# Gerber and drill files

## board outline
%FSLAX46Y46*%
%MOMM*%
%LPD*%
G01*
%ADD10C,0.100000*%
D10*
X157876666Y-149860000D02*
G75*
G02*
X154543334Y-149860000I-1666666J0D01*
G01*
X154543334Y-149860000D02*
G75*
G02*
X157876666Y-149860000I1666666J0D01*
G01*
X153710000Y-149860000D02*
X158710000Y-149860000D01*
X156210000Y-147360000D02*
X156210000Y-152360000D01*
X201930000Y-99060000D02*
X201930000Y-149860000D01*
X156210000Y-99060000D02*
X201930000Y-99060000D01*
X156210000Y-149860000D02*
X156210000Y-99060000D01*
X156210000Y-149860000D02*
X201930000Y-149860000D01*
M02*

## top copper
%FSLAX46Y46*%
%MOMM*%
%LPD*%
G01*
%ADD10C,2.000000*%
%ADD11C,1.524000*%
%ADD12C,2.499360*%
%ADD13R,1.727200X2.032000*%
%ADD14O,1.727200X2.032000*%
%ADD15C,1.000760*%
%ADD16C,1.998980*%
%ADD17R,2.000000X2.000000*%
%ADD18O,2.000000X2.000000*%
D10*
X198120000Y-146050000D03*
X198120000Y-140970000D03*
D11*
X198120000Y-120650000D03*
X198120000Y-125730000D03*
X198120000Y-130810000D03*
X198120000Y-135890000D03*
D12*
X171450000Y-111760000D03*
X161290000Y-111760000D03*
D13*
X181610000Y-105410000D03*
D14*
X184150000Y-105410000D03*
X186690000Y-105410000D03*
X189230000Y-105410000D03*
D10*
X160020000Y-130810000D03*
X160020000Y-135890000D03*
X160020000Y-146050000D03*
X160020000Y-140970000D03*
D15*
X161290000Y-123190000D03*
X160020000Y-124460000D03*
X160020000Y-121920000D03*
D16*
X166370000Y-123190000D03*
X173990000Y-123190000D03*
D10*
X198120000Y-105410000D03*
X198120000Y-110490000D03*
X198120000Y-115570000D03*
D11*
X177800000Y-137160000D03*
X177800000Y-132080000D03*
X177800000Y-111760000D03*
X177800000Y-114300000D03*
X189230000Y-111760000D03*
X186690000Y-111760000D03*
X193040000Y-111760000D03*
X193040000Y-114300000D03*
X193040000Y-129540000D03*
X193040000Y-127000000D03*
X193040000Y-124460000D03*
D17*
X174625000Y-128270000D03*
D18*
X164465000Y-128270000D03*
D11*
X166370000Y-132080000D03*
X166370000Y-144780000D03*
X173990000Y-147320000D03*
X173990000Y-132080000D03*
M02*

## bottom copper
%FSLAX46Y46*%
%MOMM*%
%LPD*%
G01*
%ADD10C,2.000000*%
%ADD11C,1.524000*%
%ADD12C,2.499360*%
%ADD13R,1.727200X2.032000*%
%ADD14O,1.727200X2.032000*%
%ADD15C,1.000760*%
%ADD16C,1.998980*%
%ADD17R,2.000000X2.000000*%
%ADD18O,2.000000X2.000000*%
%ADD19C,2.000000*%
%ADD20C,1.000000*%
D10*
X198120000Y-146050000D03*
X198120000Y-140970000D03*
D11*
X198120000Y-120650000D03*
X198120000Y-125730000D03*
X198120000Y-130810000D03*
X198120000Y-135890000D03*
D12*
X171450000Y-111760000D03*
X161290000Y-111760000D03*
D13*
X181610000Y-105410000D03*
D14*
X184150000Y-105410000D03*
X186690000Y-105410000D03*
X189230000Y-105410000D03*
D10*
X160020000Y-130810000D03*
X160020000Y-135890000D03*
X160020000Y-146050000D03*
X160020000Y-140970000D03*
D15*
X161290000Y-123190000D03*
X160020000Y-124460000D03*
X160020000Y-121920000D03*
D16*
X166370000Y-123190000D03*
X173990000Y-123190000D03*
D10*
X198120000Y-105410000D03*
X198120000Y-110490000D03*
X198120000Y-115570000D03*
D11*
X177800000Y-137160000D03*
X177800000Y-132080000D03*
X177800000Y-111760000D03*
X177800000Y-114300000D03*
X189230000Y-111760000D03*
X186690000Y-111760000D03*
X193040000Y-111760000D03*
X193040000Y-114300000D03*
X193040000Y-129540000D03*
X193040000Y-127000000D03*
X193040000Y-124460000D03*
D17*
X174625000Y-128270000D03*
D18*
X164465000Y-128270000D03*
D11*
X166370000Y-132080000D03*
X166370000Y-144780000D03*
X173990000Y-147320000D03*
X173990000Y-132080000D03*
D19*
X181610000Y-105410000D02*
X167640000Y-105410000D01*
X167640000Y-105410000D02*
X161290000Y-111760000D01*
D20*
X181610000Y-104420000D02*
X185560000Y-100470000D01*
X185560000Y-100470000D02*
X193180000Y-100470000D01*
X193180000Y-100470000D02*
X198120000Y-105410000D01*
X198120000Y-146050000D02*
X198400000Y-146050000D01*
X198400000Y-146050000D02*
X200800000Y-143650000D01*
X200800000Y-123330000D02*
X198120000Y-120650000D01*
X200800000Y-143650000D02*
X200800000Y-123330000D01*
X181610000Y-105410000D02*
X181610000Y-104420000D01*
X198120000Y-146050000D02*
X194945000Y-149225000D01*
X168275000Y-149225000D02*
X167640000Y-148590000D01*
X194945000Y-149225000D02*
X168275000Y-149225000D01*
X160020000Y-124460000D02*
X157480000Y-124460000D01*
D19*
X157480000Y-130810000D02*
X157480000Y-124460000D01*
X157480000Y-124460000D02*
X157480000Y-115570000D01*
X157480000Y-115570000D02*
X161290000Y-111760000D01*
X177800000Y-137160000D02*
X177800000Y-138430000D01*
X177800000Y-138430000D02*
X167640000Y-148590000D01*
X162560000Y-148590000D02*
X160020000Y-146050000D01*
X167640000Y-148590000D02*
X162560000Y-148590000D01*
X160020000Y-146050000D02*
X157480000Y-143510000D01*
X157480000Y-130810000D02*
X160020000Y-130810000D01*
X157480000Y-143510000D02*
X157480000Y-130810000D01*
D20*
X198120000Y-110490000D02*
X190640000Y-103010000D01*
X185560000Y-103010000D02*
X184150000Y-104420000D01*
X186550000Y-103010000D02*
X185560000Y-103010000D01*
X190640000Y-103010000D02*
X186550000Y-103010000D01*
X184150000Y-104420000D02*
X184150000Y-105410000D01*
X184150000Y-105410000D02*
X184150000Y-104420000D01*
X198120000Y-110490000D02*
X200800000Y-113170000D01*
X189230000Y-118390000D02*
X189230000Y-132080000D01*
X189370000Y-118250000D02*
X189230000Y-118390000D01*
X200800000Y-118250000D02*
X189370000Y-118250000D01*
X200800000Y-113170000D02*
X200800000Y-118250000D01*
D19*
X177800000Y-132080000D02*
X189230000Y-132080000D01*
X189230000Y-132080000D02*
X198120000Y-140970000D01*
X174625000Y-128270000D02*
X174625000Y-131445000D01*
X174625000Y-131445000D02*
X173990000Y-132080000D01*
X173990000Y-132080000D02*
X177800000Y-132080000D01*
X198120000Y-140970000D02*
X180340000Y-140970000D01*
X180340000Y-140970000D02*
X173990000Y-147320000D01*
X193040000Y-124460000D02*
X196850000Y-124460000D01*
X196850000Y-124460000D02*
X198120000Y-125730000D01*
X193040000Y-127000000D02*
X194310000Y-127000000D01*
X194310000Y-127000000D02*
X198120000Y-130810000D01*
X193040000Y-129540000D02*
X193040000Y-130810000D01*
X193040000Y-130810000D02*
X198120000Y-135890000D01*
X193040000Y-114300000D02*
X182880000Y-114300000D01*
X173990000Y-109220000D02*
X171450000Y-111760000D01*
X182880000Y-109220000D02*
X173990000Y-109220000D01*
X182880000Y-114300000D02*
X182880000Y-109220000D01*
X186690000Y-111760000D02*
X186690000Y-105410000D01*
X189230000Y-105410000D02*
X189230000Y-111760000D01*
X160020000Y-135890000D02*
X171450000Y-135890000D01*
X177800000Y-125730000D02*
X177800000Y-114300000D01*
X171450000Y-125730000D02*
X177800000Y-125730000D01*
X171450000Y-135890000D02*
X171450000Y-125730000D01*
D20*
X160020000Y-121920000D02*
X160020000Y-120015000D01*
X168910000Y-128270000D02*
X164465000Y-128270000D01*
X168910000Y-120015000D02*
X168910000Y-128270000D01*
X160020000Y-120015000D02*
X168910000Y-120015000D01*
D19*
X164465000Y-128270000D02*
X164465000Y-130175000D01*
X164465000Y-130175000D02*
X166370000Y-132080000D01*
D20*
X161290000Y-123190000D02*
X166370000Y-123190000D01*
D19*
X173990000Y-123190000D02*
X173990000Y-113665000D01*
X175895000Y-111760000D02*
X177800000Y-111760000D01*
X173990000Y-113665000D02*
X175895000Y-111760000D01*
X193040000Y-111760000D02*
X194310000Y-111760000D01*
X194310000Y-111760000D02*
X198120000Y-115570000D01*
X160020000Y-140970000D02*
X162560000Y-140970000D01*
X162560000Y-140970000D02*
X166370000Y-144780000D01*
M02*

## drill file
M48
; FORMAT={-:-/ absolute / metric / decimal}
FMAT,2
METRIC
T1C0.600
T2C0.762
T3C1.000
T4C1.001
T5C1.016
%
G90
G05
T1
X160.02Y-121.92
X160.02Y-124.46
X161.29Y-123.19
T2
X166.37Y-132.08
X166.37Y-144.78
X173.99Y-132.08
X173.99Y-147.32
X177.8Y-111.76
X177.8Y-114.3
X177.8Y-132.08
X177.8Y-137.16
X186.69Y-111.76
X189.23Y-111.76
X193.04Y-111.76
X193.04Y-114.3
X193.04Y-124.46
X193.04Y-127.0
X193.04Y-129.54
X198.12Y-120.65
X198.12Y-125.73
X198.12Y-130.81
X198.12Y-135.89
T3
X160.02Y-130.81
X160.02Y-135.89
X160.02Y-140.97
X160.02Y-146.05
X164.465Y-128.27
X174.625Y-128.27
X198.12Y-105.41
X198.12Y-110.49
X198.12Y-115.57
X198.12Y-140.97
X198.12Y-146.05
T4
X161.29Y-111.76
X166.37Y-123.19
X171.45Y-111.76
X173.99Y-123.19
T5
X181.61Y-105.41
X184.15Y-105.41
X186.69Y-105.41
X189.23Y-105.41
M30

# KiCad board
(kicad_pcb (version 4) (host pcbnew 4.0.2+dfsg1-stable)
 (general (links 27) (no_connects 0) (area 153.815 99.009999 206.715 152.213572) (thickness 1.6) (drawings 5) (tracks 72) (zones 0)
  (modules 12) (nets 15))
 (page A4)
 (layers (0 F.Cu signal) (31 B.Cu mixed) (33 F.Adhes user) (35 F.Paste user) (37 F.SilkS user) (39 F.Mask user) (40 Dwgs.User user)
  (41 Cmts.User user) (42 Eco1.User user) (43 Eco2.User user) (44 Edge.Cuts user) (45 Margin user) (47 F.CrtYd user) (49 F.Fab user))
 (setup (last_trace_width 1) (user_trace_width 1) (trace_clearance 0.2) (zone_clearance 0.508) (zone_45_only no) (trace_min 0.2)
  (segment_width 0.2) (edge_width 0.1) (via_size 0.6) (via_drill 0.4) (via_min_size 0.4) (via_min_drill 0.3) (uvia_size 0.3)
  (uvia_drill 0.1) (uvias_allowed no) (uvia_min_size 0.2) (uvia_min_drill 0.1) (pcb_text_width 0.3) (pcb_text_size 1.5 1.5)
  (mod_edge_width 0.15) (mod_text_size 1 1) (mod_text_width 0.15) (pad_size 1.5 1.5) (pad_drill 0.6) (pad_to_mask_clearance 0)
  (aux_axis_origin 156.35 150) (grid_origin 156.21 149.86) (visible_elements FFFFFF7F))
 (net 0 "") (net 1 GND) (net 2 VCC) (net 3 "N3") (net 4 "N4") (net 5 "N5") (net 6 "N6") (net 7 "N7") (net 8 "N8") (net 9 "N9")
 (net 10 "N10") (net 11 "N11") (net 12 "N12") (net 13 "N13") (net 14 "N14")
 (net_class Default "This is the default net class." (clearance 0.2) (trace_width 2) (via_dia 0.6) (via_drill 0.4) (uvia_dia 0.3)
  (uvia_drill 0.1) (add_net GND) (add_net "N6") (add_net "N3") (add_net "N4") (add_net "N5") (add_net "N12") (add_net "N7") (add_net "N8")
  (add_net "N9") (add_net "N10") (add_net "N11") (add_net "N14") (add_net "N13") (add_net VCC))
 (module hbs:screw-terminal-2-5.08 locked (layer F.Cu) (at 198.12 146.05 90)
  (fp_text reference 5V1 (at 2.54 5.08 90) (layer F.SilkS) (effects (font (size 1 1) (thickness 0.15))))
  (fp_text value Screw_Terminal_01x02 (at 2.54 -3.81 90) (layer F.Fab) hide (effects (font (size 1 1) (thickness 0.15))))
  (pad 1 thru_hole circle (at 0 0 90) (size 2 2) (drill 1) (layers *.Cu *.Mask F.SilkS) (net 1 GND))
  (pad 2 thru_hole circle (at 5.08 0 90) (size 2 2) (drill 1) (layers *.Cu *.Mask F.SilkS) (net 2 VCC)))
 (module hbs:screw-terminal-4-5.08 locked (layer F.Cu) (at 198.12 120.65 270)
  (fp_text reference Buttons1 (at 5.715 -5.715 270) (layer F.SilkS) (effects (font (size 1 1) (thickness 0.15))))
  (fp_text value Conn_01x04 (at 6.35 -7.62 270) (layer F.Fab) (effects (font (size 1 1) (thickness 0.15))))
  (pad 1 thru_hole circle (at 0 0 270) (size 1.524 1.524) (drill 0.762) (layers *.Cu *.Mask F.SilkS) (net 1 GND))
  (pad 2 thru_hole circle (at 5.08 0 270) (size 1.524 1.524) (drill 0.762) (layers *.Cu *.Mask F.SilkS) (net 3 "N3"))
  (pad 3 thru_hole circle (at 10.16 0 270) (size 1.524 1.524) (drill 0.762) (layers *.Cu *.Mask F.SilkS) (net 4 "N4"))
  (pad 4 thru_hole circle (at 15.24 0 270) (size 1.524 1.524) (drill 0.762) (layers *.Cu *.Mask F.SilkS) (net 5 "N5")))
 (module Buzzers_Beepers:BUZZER (layer F.Cu) (at 166.37 111.76)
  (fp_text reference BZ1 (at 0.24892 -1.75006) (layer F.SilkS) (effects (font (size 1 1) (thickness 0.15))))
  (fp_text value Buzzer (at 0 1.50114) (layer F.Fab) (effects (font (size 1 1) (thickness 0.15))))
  (pad 2 thru_hole circle (at 5.08 0) (size 2.49936 2.49936) (drill 1.00076) (layers *.Cu *.Mask F.SilkS) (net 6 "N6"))
  (pad 1 thru_hole circle (at -5.08 0) (size 2.49936 2.49936) (drill 1.00076) (layers *.Cu *.Mask F.SilkS) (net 1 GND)))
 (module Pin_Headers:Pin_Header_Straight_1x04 (layer F.Cu) (at 181.61 105.41 90)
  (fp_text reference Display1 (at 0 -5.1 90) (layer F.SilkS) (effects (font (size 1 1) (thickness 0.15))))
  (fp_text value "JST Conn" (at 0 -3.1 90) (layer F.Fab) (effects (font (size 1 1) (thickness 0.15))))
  (pad 1 thru_hole rect (at 0 0 90) (size 2.032 1.7272) (drill 1.016) (layers *.Cu *.Mask F.SilkS) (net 1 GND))
  (pad 2 thru_hole oval (at 0 2.54 90) (size 2.032 1.7272) (drill 1.016) (layers *.Cu *.Mask F.SilkS) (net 2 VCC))
  (pad 3 thru_hole oval (at 0 5.08 90) (size 2.032 1.7272) (drill 1.016) (layers *.Cu *.Mask F.SilkS) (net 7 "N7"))
  (pad 4 thru_hole oval (at 0 7.62 90) (size 2.032 1.7272) (drill 1.016) (layers *.Cu *.Mask F.SilkS) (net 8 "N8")))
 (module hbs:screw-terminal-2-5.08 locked (layer F.Cu) (at 160.02 130.81 270)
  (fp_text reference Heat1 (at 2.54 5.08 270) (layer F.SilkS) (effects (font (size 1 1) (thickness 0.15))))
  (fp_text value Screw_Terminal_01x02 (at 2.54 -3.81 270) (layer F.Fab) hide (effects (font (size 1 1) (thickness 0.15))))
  (pad 1 thru_hole circle (at 0 0 270) (size 2 2) (drill 1) (layers *.Cu *.Mask F.SilkS) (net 1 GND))
  (pad 2 thru_hole circle (at 5.08 0 270) (size 2 2) (drill 1) (layers *.Cu *.Mask F.SilkS) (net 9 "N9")))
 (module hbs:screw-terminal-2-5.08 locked (layer F.Cu) (at 160.02 146.05 90)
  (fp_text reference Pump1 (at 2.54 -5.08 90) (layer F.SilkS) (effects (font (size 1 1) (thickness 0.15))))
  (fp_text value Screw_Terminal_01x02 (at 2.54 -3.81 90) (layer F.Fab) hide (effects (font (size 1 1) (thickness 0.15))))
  (pad 1 thru_hole circle (at 0 0 90) (size 2 2) (drill 1) (layers *.Cu *.Mask F.SilkS) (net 1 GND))
  (pad 2 thru_hole circle (at 5.08 0 90) (size 2 2) (drill 1) (layers *.Cu *.Mask F.SilkS) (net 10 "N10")))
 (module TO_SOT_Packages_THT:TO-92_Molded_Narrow (layer F.Cu) (at 160.02 121.92 270)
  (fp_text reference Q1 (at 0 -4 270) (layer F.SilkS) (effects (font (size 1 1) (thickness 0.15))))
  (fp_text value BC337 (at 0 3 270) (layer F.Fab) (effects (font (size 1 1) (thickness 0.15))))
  (pad 2 thru_hole circle (at 1.27 -1.27) (size 1.00076 1.00076) (drill 0.6) (layers *.Cu *.Mask F.SilkS) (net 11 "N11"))
  (pad 3 thru_hole circle (at 2.54 0) (size 1.00076 1.00076) (drill 0.6) (layers *.Cu *.Mask F.SilkS) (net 1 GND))
  (pad 1 thru_hole circle (at 0 0) (size 1.00076 1.00076) (drill 0.6) (layers *.Cu *.Mask F.SilkS) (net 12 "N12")))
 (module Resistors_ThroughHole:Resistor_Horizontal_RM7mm (layer F.Cu) (at 166.37 123.19)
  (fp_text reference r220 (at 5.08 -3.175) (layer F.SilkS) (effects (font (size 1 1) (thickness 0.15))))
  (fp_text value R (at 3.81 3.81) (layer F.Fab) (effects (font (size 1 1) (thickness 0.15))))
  (pad 1 thru_hole circle (at 0 0) (size 1.99898 1.99898) (drill 1.00076) (layers *.Cu *.SilkS *.Mask) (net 11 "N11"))
  (pad 2 thru_hole circle (at 7.62 0) (size 1.99898 1.99898) (drill 1.00076) (layers *.Cu *.SilkS *.Mask) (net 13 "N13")))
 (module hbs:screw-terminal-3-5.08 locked (layer F.Cu) (at 198.12 105.41 270)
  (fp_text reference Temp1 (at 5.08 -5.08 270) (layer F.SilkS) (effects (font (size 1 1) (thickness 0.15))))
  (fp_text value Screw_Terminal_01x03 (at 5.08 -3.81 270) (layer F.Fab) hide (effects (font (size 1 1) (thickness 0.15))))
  (pad 1 thru_hole circle (at 0 0 270) (size 2 2) (drill 1) (layers *.Cu *.Mask F.SilkS) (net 1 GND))
  (pad 2 thru_hole circle (at 5.08 0 270) (size 2 2) (drill 1) (layers *.Cu *.Mask F.SilkS) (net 2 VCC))
  (pad 3 thru_hole circle (at 10.16 0 270) (size 2 2) (drill 1) (layers *.Cu *.Mask F.SilkS) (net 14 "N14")))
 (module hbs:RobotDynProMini (layer F.Cu) (at 176.53 143.51)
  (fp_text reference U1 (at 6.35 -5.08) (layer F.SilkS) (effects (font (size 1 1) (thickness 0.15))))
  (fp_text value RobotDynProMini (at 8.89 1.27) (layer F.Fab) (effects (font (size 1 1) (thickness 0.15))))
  (pad GND thru_hole circle (at 1.27 -6.35) (size 1.524 1.524) (drill 0.762) (layers *.Cu *.Mask F.SilkS) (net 1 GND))
  (pad VCC thru_hole circle (at 1.27 -11.43) (size 1.524 1.524) (drill 0.762) (layers *.Cu *.Mask F.SilkS) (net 2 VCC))
  (pad D10 thru_hole circle (at 1.27 -31.75) (size 1.524 1.524) (drill 0.762) (layers *.Cu *.Mask F.SilkS) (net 13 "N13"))
  (pad D11 thru_hole circle (at 1.27 -29.21) (size 1.524 1.524) (drill 0.762) (layers *.Cu *.Mask F.SilkS) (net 9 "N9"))
  (pad A4 thru_hole circle (at 12.7 -31.75) (size 1.524 1.524) (drill 0.762) (layers *.Cu *.Mask F.SilkS) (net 8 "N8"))
  (pad A5 thru_hole circle (at 10.16 -31.75) (size 1.524 1.524) (drill 0.762) (layers *.Cu *.Mask F.SilkS) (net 7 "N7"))
  (pad D9 thru_hole circle (at 16.51 -31.75) (size 1.524 1.524) (drill 0.762) (layers *.Cu *.Mask F.SilkS) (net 14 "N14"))
  (pad D8 thru_hole circle (at 16.51 -29.21) (size 1.524 1.524) (drill 0.762) (layers *.Cu *.Mask F.SilkS) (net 6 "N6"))
  (pad D2 thru_hole circle (at 16.51 -13.97) (size 1.524 1.524) (drill 0.762) (layers *.Cu *.Mask F.SilkS) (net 5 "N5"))
  (pad D3 thru_hole circle (at 16.51 -16.51) (size 1.524 1.524) (drill 0.762) (layers *.Cu *.Mask F.SilkS) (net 4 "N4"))
  (pad D4 thru_hole circle (at 16.51 -19.05) (size 1.524 1.524) (drill 0.762) (layers *.Cu *.Mask F.SilkS) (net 3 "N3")))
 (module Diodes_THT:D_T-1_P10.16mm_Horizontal (layer F.Cu) (at 174.625 128.27 180)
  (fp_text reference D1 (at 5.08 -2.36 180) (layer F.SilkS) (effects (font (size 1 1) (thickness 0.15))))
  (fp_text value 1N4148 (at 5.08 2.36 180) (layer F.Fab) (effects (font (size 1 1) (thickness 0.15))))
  (pad 1 thru_hole rect (at 0 0 180) (size 2 2) (drill 1) (layers *.Cu *.Mask) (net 2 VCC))
  (pad 2 thru_hole oval (at 10.16 0 180) (size 2 2) (drill 1) (layers *.Cu *.Mask) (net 12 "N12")))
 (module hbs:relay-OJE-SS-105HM (layer F.Cu) (at 166.37 132.08 270)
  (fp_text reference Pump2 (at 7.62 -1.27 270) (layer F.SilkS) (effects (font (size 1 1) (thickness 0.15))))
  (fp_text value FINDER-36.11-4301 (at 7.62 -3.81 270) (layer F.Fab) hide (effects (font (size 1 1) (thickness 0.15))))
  (pad A1 thru_hole circle (at 0 0 270) (size 1.524 1.524) (drill 0.762) (layers *.Cu *.Mask F.SilkS) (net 12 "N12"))
  (pad 14 thru_hole circle (at 12.7 0 270) (size 1.524 1.524) (drill 0.762) (layers *.Cu *.Mask F.SilkS) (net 10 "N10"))
  (pad 11 thru_hole circle (at 15.24 -7.62 270) (size 1.524 1.524) (drill 0.762) (layers *.Cu *.Mask F.SilkS) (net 2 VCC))
  (pad A2 thru_hole circle (at 0 -7.62 270) (size 1.524 1.524) (drill 0.762) (layers *.Cu *.Mask F.SilkS) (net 2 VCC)))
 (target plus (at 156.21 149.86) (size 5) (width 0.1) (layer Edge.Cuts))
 (gr_line (start 201.93 99.06) (end 201.93 149.86) (angle 90) (layer Edge.Cuts) (width 0.1))
 (gr_line (start 156.21 99.06) (end 201.93 99.06) (angle 90) (layer Edge.Cuts) (width 0.1))
 (gr_line (start 156.21 149.86) (end 156.21 99.06) (angle 90) (layer Edge.Cuts) (width 0.1))
 (gr_line (start 156.21 149.86) (end 201.93 149.86) (angle 90) (layer Edge.Cuts) (width 0.1))
 (segment (start 181.61 105.41) (end 167.64 105.41) (width 2) (layer B.Cu) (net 1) (status 10))
 (segment (start 167.64 105.41) (end 161.29 111.76) (width 2) (layer B.Cu) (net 1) (status 20))
 (segment (start 181.61 104.42) (end 185.56 100.47) (width 1) (layer B.Cu) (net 1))
 (segment (start 185.56 100.47) (end 193.18 100.47) (width 1) (layer B.Cu) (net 1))
 (segment (start 193.18 100.47) (end 198.12 105.41) (width 1) (layer B.Cu) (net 1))
 (segment (start 198.12 146.05) (end 198.4 146.05) (width 1) (layer B.Cu) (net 1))
 (segment (start 198.4 146.05) (end 200.8 143.65) (width 1) (layer B.Cu) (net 1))
 (segment (start 200.8 123.33) (end 198.12 120.65) (width 1) (layer B.Cu) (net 1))
 (segment (start 200.8 143.65) (end 200.8 123.33) (width 1) (layer B.Cu) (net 1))
 (segment (start 181.61 105.41) (end 181.61 104.42) (width 1) (layer B.Cu) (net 1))
 (segment (start 198.12 146.05) (end 194.945 149.225) (width 1) (layer B.Cu) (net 1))
 (segment (start 168.275 149.225) (end 167.64 148.59) (width 1) (layer B.Cu) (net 1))
 (segment (start 194.945 149.225) (end 168.275 149.225) (width 1) (layer B.Cu) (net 1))
 (segment (start 160.02 124.46) (end 157.48 124.46) (width 1) (layer B.Cu) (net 1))
 (segment (start 157.48 130.81) (end 157.48 124.46) (width 2) (layer B.Cu) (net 1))
 (segment (start 157.48 124.46) (end 157.48 115.57) (width 2) (layer B.Cu) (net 1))
 (segment (start 157.48 115.57) (end 161.29 111.76) (width 2) (layer B.Cu) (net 1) (status 20))
 (segment (start 177.8 137.16) (end 177.8 138.43) (width 2) (layer B.Cu) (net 1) (status 10))
 (segment (start 177.8 138.43) (end 167.64 148.59) (width 2) (layer B.Cu) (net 1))
 (segment (start 162.56 148.59) (end 160.02 146.05) (width 2) (layer B.Cu) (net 1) (status 20))
 (segment (start 167.64 148.59) (end 162.56 148.59) (width 2) (layer B.Cu) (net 1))
 (segment (start 160.02 146.05) (end 157.48 143.51) (width 2) (layer B.Cu) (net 1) (status 10))
 (segment (start 157.48 130.81) (end 160.02 130.81) (width 2) (layer B.Cu) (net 1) (status 20))
 (segment (start 157.48 143.51) (end 157.48 130.81) (width 2) (layer B.Cu) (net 1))
 (segment (start 198.12 110.49) (end 190.64 103.01) (width 1) (layer B.Cu) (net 2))
 (segment (start 185.56 103.01) (end 184.15 104.42) (width 1) (layer B.Cu) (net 2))
 (segment (start 186.55 103.01) (end 185.56 103.01) (width 1) (layer B.Cu) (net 2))
 (segment (start 190.64 103.01) (end 186.55 103.01) (width 1) (layer B.Cu) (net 2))
 (segment (start 184.15 104.42) (end 184.15 105.41) (width 1) (layer B.Cu) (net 2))
 (segment (start 184.15 105.41) (end 184.15 104.42) (width 1) (layer B.Cu) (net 2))
 (segment (start 198.12 110.49) (end 200.8 113.17) (width 1) (layer B.Cu) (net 2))
 (segment (start 189.23 118.39) (end 189.23 132.08) (width 1) (layer B.Cu) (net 2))
 (segment (start 189.37 118.25) (end 189.23 118.39) (width 1) (layer B.Cu) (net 2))
 (segment (start 200.8 118.25) (end 189.37 118.25) (width 1) (layer B.Cu) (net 2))
 (segment (start 200.8 113.17) (end 200.8 118.25) (width 1) (layer B.Cu) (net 2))
 (segment (start 177.8 132.08) (end 189.23 132.08) (width 2) (layer B.Cu) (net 2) (status 10))
 (segment (start 189.23 132.08) (end 198.12 140.97) (width 2) (layer B.Cu) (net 2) (status 20))
 (segment (start 174.625 128.27) (end 174.625 131.445) (width 2) (layer B.Cu) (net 2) (status 10))
 (segment (start 174.625 131.445) (end 173.99 132.08) (width 2) (layer B.Cu) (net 2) (status 20))
 (segment (start 173.99 132.08) (end 177.8 132.08) (width 2) (layer B.Cu) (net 2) (status 30))
 (segment (start 198.12 140.97) (end 180.34 140.97) (width 2) (layer B.Cu) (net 2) (status 10))
 (segment (start 180.34 140.97) (end 173.99 147.32) (width 2) (layer B.Cu) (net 2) (status 20))
 (segment (start 193.04 124.46) (end 196.85 124.46) (width 2) (layer B.Cu) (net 3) (status 10))
 (segment (start 196.85 124.46) (end 198.12 125.73) (width 2) (layer B.Cu) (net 3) (status 20))
 (segment (start 193.04 127) (end 194.31 127) (width 2) (layer B.Cu) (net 4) (status 10))
 (segment (start 194.31 127) (end 198.12 130.81) (width 2) (layer B.Cu) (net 4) (status 20))
 (segment (start 193.04 129.54) (end 193.04 130.81) (width 2) (layer B.Cu) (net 5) (status 10))
 (segment (start 193.04 130.81) (end 198.12 135.89) (width 2) (layer B.Cu) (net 5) (status 20))
 (segment (start 193.04 114.3) (end 182.88 114.3) (width 2) (layer B.Cu) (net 6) (status 10))
 (segment (start 173.99 109.22) (end 171.45 111.76) (width 2) (layer B.Cu) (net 6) (status 20))
 (segment (start 182.88 109.22) (end 173.99 109.22) (width 2) (layer B.Cu) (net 6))
 (segment (start 182.88 114.3) (end 182.88 109.22) (width 2) (layer B.Cu) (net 6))
 (segment (start 186.69 111.76) (end 186.69 105.41) (width 2) (layer B.Cu) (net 7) (status 30))
 (segment (start 189.23 105.41) (end 189.23 111.76) (width 2) (layer B.Cu) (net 8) (status 30))
 (segment (start 160.02 135.89) (end 171.45 135.89) (width 2) (layer B.Cu) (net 9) (status 10))
 (segment (start 177.8 125.73) (end 177.8 114.3) (width 2) (layer B.Cu) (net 9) (status 20))
 (segment (start 171.45 125.73) (end 177.8 125.73) (width 2) (layer B.Cu) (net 9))
 (segment (start 171.45 135.89) (end 171.45 125.73) (width 2) (layer B.Cu) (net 9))
 (segment (start 160.02 121.92) (end 160.02 120.015) (width 1) (layer B.Cu) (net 12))
 (segment (start 168.91 128.27) (end 164.465 128.27) (width 1) (layer B.Cu) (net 12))
 (segment (start 168.91 120.015) (end 168.91 128.27) (width 1) (layer B.Cu) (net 12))
 (segment (start 160.02 120.015) (end 168.91 120.015) (width 1) (layer B.Cu) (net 12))
 (segment (start 164.465 128.27) (end 164.465 130.175) (width 2) (layer B.Cu) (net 12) (status 10))
 (segment (start 164.465 130.175) (end 166.37 132.08) (width 2) (layer B.Cu) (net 12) (status 20))
 (segment (start 161.29 123.19) (end 166.37 123.19) (width 1) (layer B.Cu) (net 11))
 (segment (start 173.99 123.19) (end 173.99 113.665) (width 2) (layer B.Cu) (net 13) (status 10))
 (segment (start 175.895 111.76) (end 177.8 111.76) (width 2) (layer B.Cu) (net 13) (status 20))
 (segment (start 173.99 113.665) (end 175.895 111.76) (width 2) (layer B.Cu) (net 13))
 (segment (start 193.04 111.76) (end 194.31 111.76) (width 2) (layer B.Cu) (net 14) (status 10))
 (segment (start 194.31 111.76) (end 198.12 115.57) (width 2) (layer B.Cu) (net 14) (status 20))
 (segment (start 160.02 140.97) (end 162.56 140.97) (width 2) (layer B.Cu) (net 10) (status 10))
 (segment (start 162.56 140.97) (end 166.37 144.78) (width 2) (layer B.Cu) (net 10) (status 20)))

